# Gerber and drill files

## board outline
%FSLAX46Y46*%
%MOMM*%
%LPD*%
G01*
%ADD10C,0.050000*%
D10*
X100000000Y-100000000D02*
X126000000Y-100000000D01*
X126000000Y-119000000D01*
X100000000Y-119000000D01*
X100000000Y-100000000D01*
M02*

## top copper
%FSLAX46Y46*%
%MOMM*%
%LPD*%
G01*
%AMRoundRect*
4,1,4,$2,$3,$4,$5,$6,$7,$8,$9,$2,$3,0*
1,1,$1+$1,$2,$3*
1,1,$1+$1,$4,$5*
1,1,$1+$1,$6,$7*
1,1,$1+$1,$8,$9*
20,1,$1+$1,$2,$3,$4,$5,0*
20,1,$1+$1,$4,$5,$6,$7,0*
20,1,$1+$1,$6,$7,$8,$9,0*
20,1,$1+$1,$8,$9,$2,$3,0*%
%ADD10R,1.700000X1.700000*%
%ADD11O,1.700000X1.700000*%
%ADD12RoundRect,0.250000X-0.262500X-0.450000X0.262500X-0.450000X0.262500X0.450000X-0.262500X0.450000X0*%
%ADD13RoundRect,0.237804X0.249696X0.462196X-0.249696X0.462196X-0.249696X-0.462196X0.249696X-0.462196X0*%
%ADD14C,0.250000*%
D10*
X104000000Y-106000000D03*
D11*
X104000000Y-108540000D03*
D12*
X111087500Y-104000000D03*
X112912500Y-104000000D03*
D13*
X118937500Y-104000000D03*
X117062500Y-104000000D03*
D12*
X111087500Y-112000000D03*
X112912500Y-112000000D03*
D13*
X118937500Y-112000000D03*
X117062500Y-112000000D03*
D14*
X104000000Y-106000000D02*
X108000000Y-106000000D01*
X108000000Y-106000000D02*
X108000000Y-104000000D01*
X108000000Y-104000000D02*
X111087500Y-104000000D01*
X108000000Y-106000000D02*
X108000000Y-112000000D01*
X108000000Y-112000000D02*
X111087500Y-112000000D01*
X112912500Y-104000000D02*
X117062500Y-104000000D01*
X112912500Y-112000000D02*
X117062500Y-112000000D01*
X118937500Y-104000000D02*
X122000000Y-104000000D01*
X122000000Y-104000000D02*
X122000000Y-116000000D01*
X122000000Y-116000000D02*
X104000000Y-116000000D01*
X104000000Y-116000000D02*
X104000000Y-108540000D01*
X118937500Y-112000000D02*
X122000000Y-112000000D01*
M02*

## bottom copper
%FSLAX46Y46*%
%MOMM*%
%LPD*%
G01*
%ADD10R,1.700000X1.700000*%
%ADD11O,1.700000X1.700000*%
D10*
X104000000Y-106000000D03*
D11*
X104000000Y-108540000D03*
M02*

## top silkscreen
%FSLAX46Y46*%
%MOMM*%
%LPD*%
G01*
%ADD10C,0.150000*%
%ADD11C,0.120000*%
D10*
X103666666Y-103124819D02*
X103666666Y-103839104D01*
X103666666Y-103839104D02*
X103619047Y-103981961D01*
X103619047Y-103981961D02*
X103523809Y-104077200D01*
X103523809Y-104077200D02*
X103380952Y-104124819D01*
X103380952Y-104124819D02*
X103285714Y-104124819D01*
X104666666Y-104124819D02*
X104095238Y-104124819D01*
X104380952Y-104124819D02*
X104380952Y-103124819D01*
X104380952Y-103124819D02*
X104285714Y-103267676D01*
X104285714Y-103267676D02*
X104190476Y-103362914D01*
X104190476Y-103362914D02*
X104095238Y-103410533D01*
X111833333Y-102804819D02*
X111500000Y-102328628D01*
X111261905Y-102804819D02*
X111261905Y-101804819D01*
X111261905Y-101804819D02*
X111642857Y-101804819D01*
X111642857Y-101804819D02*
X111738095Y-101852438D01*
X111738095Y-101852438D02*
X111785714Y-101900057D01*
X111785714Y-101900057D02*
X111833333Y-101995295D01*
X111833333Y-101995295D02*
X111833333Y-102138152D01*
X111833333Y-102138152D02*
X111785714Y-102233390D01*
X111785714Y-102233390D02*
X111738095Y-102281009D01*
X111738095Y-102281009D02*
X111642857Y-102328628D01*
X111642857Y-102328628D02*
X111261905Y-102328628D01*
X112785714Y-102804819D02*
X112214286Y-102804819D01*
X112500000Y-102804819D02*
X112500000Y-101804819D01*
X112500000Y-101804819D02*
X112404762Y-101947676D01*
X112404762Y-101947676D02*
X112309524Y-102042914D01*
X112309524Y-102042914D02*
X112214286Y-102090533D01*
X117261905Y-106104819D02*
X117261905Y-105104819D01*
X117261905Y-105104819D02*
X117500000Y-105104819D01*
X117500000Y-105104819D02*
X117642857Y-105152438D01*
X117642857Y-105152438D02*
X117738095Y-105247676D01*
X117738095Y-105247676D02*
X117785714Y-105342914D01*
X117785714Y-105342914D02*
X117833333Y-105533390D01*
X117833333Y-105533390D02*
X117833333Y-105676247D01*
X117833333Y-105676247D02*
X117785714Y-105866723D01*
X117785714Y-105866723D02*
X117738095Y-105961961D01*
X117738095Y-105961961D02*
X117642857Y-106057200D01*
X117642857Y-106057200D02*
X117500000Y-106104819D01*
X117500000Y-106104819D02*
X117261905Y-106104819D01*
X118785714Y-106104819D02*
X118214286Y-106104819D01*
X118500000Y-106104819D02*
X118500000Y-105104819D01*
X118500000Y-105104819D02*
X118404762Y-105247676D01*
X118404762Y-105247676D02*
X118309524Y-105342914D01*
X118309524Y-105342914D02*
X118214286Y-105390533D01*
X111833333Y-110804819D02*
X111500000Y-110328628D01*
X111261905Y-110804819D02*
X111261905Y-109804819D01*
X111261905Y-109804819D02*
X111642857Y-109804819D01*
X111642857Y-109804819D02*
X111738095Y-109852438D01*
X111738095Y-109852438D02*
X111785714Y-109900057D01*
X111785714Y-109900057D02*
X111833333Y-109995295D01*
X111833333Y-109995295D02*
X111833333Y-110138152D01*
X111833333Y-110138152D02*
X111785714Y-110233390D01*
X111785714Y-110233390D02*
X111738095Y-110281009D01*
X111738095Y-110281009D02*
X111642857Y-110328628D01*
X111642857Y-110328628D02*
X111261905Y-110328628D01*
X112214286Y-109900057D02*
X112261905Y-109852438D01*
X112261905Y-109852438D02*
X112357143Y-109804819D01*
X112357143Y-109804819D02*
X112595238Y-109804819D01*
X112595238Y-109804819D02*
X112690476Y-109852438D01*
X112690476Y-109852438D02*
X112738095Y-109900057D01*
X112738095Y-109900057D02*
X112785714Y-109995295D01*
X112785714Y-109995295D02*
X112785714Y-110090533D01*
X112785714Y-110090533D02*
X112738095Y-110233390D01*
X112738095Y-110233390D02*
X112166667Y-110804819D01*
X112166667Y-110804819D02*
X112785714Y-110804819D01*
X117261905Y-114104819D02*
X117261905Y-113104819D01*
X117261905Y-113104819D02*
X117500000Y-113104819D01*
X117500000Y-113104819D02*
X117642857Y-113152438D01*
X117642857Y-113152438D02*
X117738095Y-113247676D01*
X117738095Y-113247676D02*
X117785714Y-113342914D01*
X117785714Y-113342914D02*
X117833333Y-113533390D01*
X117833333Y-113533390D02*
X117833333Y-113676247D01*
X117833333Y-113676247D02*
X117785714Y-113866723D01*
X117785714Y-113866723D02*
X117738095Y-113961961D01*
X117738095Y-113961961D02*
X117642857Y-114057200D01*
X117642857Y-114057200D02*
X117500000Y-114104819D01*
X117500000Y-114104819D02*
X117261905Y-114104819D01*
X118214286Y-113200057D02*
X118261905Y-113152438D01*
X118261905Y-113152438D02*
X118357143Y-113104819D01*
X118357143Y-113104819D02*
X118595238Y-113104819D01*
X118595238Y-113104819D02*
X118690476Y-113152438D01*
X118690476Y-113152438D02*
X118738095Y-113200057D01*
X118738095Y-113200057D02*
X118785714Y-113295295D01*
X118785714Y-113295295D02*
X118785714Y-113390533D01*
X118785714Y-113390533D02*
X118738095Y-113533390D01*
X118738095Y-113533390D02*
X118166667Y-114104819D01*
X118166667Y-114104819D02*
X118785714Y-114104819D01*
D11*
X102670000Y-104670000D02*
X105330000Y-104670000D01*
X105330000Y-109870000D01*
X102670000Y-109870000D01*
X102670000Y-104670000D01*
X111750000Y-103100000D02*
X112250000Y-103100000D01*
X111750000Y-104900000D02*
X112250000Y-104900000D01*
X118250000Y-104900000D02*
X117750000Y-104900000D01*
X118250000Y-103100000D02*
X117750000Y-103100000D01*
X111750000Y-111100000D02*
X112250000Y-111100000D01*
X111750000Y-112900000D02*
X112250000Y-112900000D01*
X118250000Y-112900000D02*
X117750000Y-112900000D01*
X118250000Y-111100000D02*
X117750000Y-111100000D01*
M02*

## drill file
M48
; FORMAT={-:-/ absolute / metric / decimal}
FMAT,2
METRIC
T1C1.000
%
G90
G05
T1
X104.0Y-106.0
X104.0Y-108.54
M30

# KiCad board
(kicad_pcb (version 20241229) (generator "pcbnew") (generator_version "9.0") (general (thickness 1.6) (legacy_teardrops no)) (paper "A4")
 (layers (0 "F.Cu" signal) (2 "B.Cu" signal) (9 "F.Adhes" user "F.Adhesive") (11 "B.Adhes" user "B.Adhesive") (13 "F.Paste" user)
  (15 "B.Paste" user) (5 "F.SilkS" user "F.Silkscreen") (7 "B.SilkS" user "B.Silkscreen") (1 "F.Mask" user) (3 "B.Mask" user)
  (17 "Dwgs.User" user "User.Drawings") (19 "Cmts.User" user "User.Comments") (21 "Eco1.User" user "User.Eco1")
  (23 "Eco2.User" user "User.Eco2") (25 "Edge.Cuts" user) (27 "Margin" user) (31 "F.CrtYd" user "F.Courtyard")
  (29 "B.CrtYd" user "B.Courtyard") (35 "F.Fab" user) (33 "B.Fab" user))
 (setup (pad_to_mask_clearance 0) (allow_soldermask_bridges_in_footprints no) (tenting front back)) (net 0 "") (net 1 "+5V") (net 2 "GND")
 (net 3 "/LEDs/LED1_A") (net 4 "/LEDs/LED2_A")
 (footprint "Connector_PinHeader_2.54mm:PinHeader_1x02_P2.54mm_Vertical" (layer "F.Cu") (at 104 106)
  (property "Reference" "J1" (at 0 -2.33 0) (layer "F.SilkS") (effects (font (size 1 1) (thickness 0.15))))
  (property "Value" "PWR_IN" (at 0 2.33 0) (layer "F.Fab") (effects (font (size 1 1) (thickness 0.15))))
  (fp_rect (start -1.33 -1.33) (end 1.33 3.87) (stroke (width 0.12) (type solid)) (fill no) (layer "F.SilkS"))
  (pad "1" thru_hole rect (at 0 0) (size 1.7 1.7) (drill 1) (layers "*.Cu" "*.Mask") (remove_unused_layers no) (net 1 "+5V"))
  (pad "2" thru_hole oval (at 0 2.54) (size 1.7 1.7) (drill 1) (layers "*.Cu" "*.Mask") (remove_unused_layers no) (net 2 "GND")))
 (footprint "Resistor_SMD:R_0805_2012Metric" (layer "F.Cu") (at 112 104)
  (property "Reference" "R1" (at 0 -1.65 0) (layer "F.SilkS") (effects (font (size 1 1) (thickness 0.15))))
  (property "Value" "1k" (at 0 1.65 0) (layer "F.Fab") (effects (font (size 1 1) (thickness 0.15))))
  (fp_line (start -0.25 -0.9) (end 0.25 -0.9) (stroke (width 0.12) (type solid)) (layer "F.SilkS"))
  (fp_line (start -0.25 0.9) (end 0.25 0.9) (stroke (width 0.12) (type solid)) (layer "F.SilkS"))
  (pad "1" smd roundrect (at -0.9125 0) (size 1.025 1.4) (layers "F.Cu" "F.Mask" "F.Paste") (roundrect_rratio 0.243902) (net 1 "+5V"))
  (pad "2" smd roundrect (at 0.9125 0) (size 1.025 1.4) (layers "F.Cu" "F.Mask" "F.Paste") (roundrect_rratio 0.243902)
   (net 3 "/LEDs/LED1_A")))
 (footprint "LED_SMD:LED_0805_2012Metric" (layer "F.Cu") (at 118 104 180)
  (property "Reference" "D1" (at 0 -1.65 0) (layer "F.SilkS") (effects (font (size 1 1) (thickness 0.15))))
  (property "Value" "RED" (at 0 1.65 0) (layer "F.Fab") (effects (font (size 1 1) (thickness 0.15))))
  (fp_line (start -0.25 -0.9) (end 0.25 -0.9) (stroke (width 0.12) (type solid)) (layer "F.SilkS"))
  (fp_line (start -0.25 0.9) (end 0.25 0.9) (stroke (width 0.12) (type solid)) (layer "F.SilkS"))
  (pad "1" smd roundrect (at -0.9375 0 180) (size 0.975 1.4) (layers "F.Cu" "F.Mask" "F.Paste") (roundrect_rratio 0.243902) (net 2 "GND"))
  (pad "2" smd roundrect (at 0.9375 0 180) (size 0.975 1.4) (layers "F.Cu" "F.Mask" "F.Paste") (roundrect_rratio 0.243902)
   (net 3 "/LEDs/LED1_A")))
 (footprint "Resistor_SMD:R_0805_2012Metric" (layer "F.Cu") (at 112 112)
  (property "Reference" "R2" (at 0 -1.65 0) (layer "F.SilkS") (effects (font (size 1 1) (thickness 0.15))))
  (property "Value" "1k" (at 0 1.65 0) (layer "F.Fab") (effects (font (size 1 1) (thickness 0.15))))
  (fp_line (start -0.25 -0.9) (end 0.25 -0.9) (stroke (width 0.12) (type solid)) (layer "F.SilkS"))
  (fp_line (start -0.25 0.9) (end 0.25 0.9) (stroke (width 0.12) (type solid)) (layer "F.SilkS"))
  (pad "1" smd roundrect (at -0.9125 0) (size 1.025 1.4) (layers "F.Cu" "F.Mask" "F.Paste") (roundrect_rratio 0.243902) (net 1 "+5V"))
  (pad "2" smd roundrect (at 0.9125 0) (size 1.025 1.4) (layers "F.Cu" "F.Mask" "F.Paste") (roundrect_rratio 0.243902)
   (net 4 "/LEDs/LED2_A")))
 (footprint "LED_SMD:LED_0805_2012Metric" (layer "F.Cu") (at 118 112 180)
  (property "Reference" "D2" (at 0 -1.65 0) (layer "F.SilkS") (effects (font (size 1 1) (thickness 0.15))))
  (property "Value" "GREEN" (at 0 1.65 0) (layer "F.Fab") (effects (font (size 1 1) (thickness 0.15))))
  (fp_line (start -0.25 -0.9) (end 0.25 -0.9) (stroke (width 0.12) (type solid)) (layer "F.SilkS"))
  (fp_line (start -0.25 0.9) (end 0.25 0.9) (stroke (width 0.12) (type solid)) (layer "F.SilkS"))
  (pad "1" smd roundrect (at -0.9375 0 180) (size 0.975 1.4) (layers "F.Cu" "F.Mask" "F.Paste") (roundrect_rratio 0.243902) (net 2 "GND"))
  (pad "2" smd roundrect (at 0.9375 0 180) (size 0.975 1.4) (layers "F.Cu" "F.Mask" "F.Paste") (roundrect_rratio 0.243902)
   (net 4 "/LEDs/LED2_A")))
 (gr_rect (start 100 100) (end 126 119) (stroke (width 0.05) (type default)) (fill no) (layer "Edge.Cuts"))
 (segment (start 104 106) (end 108 106) (width 0.25) (layer "F.Cu") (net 1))
 (segment (start 108 106) (end 108 104) (width 0.25) (layer "F.Cu") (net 1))
 (segment (start 108 104) (end 111.0875 104) (width 0.25) (layer "F.Cu") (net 1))
 (segment (start 108 106) (end 108 112) (width 0.25) (layer "F.Cu") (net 1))
 (segment (start 108 112) (end 111.0875 112) (width 0.25) (layer "F.Cu") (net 1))
 (segment (start 112.9125 104) (end 117.0625 104) (width 0.25) (layer "F.Cu") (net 3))
 (segment (start 112.9125 112) (end 117.0625 112) (width 0.25) (layer "F.Cu") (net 4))
 (segment (start 118.9375 104) (end 122 104) (width 0.25) (layer "F.Cu") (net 2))
 (segment (start 122 104) (end 122 116) (width 0.25) (layer "F.Cu") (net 2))
 (segment (start 122 116) (end 104 116) (width 0.25) (layer "F.Cu") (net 2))
 (segment (start 104 116) (end 104 108.54) (width 0.25) (layer "F.Cu") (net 2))
 (segment (start 118.9375 112) (end 122 112) (width 0.25) (layer "F.Cu") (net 2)))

